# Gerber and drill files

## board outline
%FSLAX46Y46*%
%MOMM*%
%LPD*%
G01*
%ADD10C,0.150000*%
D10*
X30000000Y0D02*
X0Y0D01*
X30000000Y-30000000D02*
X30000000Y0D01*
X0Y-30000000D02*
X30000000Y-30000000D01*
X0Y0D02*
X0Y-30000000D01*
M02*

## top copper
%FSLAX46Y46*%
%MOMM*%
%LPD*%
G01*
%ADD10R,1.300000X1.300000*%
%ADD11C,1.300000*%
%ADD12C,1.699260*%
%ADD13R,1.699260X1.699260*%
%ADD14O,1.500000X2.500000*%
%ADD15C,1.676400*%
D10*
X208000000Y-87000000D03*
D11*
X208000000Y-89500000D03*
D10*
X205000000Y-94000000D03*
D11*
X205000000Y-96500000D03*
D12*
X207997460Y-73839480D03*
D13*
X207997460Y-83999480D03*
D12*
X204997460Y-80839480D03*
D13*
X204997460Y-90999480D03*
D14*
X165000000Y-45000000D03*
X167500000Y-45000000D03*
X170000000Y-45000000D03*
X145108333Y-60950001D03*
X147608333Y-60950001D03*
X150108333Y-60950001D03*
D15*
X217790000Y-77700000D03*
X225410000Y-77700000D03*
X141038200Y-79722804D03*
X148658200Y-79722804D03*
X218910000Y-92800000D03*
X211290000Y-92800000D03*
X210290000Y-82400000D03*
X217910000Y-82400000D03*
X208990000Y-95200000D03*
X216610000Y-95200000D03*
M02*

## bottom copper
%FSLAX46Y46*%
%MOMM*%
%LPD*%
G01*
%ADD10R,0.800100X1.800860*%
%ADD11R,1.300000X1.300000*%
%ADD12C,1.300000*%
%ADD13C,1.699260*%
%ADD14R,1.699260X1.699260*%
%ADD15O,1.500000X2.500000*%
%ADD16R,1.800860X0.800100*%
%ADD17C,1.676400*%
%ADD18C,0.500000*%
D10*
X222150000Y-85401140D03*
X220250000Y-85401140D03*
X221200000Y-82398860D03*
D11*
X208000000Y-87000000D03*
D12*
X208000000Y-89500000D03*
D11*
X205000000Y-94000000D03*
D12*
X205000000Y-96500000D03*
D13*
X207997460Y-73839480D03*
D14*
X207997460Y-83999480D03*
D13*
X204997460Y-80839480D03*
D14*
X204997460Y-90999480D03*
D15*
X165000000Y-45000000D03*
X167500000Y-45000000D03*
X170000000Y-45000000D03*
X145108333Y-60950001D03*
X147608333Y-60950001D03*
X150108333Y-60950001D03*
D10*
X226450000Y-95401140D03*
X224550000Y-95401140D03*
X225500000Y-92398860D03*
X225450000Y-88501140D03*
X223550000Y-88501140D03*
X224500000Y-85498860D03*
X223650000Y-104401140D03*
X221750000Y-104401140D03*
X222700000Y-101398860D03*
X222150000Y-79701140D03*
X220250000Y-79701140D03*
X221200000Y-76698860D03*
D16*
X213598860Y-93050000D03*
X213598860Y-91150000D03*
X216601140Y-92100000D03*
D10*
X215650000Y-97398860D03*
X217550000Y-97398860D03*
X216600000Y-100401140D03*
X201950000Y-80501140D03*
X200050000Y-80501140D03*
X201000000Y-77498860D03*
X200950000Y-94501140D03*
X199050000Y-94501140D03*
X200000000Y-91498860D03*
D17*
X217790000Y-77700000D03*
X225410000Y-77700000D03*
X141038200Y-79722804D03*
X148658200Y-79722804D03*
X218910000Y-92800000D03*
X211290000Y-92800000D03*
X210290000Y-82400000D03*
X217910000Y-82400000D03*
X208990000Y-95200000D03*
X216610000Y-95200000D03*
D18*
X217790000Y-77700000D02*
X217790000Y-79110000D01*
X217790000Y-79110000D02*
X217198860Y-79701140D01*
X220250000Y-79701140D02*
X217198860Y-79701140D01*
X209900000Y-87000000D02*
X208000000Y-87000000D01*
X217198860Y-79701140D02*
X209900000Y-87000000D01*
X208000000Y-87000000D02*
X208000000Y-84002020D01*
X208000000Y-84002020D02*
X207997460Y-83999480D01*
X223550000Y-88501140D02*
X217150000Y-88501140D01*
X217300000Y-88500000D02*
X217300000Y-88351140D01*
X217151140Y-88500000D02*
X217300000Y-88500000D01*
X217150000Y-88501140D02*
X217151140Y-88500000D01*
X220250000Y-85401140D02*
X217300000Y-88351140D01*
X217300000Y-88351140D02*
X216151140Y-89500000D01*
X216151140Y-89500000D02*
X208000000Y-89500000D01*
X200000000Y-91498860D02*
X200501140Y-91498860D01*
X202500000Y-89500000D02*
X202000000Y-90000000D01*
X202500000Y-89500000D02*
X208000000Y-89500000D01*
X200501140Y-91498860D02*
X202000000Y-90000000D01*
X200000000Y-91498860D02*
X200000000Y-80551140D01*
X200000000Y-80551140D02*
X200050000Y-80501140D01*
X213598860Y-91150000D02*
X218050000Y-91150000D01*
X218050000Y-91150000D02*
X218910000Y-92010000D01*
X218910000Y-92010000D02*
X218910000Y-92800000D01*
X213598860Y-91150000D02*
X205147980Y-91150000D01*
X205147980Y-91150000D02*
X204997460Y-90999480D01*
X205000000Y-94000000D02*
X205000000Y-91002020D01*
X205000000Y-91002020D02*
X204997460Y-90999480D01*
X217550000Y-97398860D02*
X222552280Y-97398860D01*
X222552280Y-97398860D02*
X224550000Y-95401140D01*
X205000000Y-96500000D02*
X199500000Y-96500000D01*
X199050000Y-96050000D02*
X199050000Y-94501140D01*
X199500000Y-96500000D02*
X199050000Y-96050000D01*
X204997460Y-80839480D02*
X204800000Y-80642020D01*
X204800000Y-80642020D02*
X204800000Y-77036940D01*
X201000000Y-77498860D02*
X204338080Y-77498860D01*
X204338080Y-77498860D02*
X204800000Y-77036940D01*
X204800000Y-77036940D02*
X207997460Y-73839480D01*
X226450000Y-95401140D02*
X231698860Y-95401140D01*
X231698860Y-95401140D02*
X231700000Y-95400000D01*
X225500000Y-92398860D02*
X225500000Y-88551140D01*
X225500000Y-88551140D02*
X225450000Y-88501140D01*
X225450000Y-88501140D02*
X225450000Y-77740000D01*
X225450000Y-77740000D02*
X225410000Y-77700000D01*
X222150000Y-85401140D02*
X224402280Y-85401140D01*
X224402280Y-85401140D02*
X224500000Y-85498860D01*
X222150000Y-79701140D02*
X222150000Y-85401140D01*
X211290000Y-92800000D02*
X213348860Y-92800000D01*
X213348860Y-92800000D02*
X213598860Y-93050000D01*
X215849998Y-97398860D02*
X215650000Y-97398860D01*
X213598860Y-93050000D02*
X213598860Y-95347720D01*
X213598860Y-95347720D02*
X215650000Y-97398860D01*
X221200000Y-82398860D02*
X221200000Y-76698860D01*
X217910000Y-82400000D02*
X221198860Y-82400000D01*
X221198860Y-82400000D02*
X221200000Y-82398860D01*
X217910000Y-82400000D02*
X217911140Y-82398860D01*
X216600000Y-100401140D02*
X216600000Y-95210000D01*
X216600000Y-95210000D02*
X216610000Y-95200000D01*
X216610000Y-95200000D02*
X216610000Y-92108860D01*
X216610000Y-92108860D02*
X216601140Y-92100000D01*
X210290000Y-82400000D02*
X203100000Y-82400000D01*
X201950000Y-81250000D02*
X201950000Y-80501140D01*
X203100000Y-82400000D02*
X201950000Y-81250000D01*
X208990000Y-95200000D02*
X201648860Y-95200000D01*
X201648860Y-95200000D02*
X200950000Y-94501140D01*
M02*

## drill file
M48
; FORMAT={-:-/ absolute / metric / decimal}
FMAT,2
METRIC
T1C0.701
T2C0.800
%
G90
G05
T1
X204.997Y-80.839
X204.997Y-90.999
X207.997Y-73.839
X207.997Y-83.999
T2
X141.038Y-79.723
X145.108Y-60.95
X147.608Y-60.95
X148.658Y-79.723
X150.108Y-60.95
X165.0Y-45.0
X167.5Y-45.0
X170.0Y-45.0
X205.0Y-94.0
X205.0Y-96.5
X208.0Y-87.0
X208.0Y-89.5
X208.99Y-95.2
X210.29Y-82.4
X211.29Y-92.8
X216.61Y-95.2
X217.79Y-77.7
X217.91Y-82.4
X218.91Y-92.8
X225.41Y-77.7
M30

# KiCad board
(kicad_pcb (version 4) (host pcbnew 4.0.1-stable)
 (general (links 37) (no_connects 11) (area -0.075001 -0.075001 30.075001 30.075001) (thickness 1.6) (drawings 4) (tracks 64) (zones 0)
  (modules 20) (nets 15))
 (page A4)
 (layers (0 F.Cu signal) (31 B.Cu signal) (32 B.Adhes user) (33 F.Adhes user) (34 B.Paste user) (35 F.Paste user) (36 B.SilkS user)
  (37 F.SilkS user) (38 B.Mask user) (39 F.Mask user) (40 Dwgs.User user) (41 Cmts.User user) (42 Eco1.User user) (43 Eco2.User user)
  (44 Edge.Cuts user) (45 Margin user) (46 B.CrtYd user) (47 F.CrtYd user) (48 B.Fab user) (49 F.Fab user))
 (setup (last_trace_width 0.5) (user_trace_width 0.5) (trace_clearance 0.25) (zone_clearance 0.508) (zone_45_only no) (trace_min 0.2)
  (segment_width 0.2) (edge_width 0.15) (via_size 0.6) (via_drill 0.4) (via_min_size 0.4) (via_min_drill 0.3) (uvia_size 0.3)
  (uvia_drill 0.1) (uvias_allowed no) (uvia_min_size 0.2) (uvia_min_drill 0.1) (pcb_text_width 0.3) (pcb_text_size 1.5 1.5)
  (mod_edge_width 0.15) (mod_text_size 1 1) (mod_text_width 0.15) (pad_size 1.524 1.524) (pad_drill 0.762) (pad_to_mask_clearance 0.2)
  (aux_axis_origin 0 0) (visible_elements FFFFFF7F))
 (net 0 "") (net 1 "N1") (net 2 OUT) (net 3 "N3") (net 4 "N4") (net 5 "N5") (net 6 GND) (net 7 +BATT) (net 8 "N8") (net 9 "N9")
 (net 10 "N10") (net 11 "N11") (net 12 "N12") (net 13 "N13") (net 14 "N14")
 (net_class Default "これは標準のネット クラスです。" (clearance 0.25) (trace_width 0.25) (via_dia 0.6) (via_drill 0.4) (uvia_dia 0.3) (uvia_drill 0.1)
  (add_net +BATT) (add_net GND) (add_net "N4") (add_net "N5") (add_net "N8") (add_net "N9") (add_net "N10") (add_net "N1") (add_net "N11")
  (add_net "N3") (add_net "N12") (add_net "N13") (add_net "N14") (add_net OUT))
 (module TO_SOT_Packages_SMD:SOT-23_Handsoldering (layer B.Cu) (at 221.2 83.9 180)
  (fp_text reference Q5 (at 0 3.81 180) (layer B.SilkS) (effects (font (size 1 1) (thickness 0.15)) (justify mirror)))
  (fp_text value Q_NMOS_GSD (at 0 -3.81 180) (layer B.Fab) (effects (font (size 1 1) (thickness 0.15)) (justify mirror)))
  (pad 1 smd rect (at -0.95 -1.50114 180) (size 0.8001 1.80086) (layers B.Cu B.Paste B.Mask) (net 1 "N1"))
  (pad 2 smd rect (at 0.95 -1.50114 180) (size 0.8001 1.80086) (layers B.Cu B.Paste B.Mask) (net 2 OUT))
  (pad 3 smd rect (at 0 1.50114 180) (size 0.8001 1.80086) (layers B.Cu B.Paste B.Mask) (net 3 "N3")))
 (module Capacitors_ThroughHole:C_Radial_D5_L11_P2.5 (layer F.Cu) (at 208 87 270)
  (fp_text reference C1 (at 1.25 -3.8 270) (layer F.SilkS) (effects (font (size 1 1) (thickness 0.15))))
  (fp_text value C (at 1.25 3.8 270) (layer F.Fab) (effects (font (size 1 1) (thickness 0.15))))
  (pad 1 thru_hole rect (at 0 0 270) (size 1.3 1.3) (drill 0.8) (layers *.Cu *.Mask F.SilkS) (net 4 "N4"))
  (pad 2 thru_hole circle (at 2.5 0 270) (size 1.3 1.3) (drill 0.8) (layers *.Cu *.Mask F.SilkS) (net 2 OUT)))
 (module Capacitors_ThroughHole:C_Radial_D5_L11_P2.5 (layer F.Cu) (at 205 94 270)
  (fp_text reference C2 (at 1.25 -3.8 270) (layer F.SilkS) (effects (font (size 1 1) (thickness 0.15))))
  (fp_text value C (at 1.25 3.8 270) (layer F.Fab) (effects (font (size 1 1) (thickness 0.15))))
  (pad 1 thru_hole rect (at 0 0 270) (size 1.3 1.3) (drill 0.8) (layers *.Cu *.Mask F.SilkS) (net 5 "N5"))
  (pad 2 thru_hole circle (at 2.5 0 270) (size 1.3 1.3) (drill 0.8) (layers *.Cu *.Mask F.SilkS) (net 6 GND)))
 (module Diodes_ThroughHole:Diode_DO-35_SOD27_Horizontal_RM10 (layer F.Cu) (at 208 84 90)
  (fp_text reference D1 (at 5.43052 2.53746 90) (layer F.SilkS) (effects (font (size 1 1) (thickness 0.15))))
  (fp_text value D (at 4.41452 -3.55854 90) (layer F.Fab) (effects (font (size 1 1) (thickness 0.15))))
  (pad 2 thru_hole circle (at 10.16052 -0.00254 270) (size 1.69926 1.69926) (drill 0.70104) (layers *.Cu *.Mask F.SilkS) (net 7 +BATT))
  (pad 1 thru_hole rect (at 0.00052 -0.00254 270) (size 1.69926 1.69926) (drill 0.70104) (layers *.Cu *.Mask F.SilkS) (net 4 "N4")))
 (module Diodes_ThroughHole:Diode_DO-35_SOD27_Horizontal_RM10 (layer F.Cu) (at 205 91 90)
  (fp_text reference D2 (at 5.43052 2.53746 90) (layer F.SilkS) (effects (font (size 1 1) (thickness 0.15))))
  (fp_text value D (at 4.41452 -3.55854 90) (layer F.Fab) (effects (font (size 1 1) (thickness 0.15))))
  (pad 2 thru_hole circle (at 10.16052 -0.00254 270) (size 1.69926 1.69926) (drill 0.70104) (layers *.Cu *.Mask F.SilkS) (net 7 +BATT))
  (pad 1 thru_hole rect (at 0.00052 -0.00254 270) (size 1.69926 1.69926) (drill 0.70104) (layers *.Cu *.Mask F.SilkS) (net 5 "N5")))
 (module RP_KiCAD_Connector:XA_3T (layer F.Cu) (at 165 45)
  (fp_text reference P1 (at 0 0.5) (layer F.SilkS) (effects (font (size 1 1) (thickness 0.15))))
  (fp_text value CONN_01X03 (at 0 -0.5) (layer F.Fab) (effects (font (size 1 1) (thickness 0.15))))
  (pad 1 thru_hole oval (at 0 0) (size 1.5 2.5) (drill 0.8) (layers *.Cu *.Mask F.SilkS) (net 6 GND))
  (pad 2 thru_hole oval (at 2.5 0) (size 1.5 2.5) (drill 0.8) (layers *.Cu *.Mask F.SilkS) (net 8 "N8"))
  (pad 3 thru_hole oval (at 5 0) (size 1.5 2.5) (drill 0.8) (layers *.Cu *.Mask F.SilkS) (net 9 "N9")))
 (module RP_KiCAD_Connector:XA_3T (layer F.Cu) (at 145.108333 60.950001)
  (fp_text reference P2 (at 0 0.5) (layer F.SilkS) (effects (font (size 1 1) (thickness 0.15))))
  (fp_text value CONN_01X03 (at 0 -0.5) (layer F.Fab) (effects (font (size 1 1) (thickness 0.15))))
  (pad 1 thru_hole oval (at 0 0) (size 1.5 2.5) (drill 0.8) (layers *.Cu *.Mask F.SilkS) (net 6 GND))
  (pad 2 thru_hole oval (at 2.5 0) (size 1.5 2.5) (drill 0.8) (layers *.Cu *.Mask F.SilkS) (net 7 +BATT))
  (pad 3 thru_hole oval (at 5 0) (size 1.5 2.5) (drill 0.8) (layers *.Cu *.Mask F.SilkS) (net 2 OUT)))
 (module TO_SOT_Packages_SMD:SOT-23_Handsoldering (layer B.Cu) (at 225.5 93.9 180)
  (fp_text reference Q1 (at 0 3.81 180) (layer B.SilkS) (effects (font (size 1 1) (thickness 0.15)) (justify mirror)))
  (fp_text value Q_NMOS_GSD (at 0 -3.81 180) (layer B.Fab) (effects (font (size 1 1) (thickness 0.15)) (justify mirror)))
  (pad 1 smd rect (at -0.95 -1.50114 180) (size 0.8001 1.80086) (layers B.Cu B.Paste B.Mask) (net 9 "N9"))
  (pad 2 smd rect (at 0.95 -1.50114 180) (size 0.8001 1.80086) (layers B.Cu B.Paste B.Mask) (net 6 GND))
  (pad 3 smd rect (at 0 1.50114 180) (size 0.8001 1.80086) (layers B.Cu B.Paste B.Mask) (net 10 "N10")))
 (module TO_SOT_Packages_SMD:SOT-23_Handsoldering (layer B.Cu) (at 224.5 87 180)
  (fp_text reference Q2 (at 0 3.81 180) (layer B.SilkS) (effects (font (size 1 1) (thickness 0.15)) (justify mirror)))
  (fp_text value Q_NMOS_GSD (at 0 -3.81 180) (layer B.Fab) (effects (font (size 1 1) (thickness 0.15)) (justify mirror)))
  (pad 1 smd rect (at -0.95 -1.50114 180) (size 0.8001 1.80086) (layers B.Cu B.Paste B.Mask) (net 10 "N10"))
  (pad 2 smd rect (at 0.95 -1.50114 180) (size 0.8001 1.80086) (layers B.Cu B.Paste B.Mask) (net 2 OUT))
  (pad 3 smd rect (at 0 1.50114 180) (size 0.8001 1.80086) (layers B.Cu B.Paste B.Mask) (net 1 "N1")))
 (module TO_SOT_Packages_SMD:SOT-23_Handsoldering (layer B.Cu) (at 222.7 102.9 180)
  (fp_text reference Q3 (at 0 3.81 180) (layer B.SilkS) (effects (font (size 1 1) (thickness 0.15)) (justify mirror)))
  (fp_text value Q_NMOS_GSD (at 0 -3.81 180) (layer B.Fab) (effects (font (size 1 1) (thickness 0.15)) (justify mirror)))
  (pad 1 smd rect (at -0.95 -1.50114 180) (size 0.8001 1.80086) (layers B.Cu B.Paste B.Mask) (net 8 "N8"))
  (pad 2 smd rect (at 0.95 -1.50114 180) (size 0.8001 1.80086) (layers B.Cu B.Paste B.Mask) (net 6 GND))
  (pad 3 smd rect (at 0 1.50114 180) (size 0.8001 1.80086) (layers B.Cu B.Paste B.Mask) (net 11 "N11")))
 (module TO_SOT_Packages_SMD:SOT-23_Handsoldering (layer B.Cu) (at 221.2 78.2 180)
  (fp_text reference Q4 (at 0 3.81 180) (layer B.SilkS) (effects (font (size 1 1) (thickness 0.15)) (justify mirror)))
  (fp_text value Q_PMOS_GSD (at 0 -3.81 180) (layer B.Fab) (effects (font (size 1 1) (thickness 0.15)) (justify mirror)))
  (pad 1 smd rect (at -0.95 -1.50114 180) (size 0.8001 1.80086) (layers B.Cu B.Paste B.Mask) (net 1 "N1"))
  (pad 2 smd rect (at 0.95 -1.50114 180) (size 0.8001 1.80086) (layers B.Cu B.Paste B.Mask) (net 4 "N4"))
  (pad 3 smd rect (at 0 1.50114 180) (size 0.8001 1.80086) (layers B.Cu B.Paste B.Mask) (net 3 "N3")))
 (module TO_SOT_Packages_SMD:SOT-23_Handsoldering (layer B.Cu) (at 215.1 92.1 90)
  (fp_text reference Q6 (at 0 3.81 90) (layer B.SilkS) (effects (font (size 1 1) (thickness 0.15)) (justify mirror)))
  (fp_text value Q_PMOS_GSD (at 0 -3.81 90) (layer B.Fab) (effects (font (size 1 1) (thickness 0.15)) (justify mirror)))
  (pad 1 smd rect (at -0.95 -1.50114 90) (size 0.8001 1.80086) (layers B.Cu B.Paste B.Mask) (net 11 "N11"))
  (pad 2 smd rect (at 0.95 -1.50114 90) (size 0.8001 1.80086) (layers B.Cu B.Paste B.Mask) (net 5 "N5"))
  (pad 3 smd rect (at 0 1.50114 90) (size 0.8001 1.80086) (layers B.Cu B.Paste B.Mask) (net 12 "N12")))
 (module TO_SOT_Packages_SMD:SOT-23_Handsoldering (layer B.Cu) (at 216.6 98.9)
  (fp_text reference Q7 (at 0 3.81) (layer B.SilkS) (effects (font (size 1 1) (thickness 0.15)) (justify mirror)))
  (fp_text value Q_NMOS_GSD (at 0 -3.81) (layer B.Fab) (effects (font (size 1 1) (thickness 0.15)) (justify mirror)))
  (pad 1 smd rect (at -0.95 -1.50114) (size 0.8001 1.80086) (layers B.Cu B.Paste B.Mask) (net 11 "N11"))
  (pad 2 smd rect (at 0.95 -1.50114) (size 0.8001 1.80086) (layers B.Cu B.Paste B.Mask) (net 6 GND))
  (pad 3 smd rect (at 0 1.50114) (size 0.8001 1.80086) (layers B.Cu B.Paste B.Mask) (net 12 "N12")))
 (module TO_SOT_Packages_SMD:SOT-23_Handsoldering (layer B.Cu) (at 201 79 180)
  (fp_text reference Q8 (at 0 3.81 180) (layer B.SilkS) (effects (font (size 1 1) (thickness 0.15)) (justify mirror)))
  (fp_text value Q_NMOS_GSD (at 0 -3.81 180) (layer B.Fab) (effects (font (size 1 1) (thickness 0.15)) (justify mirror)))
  (pad 1 smd rect (at -0.95 -1.50114 180) (size 0.8001 1.80086) (layers B.Cu B.Paste B.Mask) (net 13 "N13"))
  (pad 2 smd rect (at 0.95 -1.50114 180) (size 0.8001 1.80086) (layers B.Cu B.Paste B.Mask) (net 2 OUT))
  (pad 3 smd rect (at 0 1.50114 180) (size 0.8001 1.80086) (layers B.Cu B.Paste B.Mask) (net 7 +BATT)))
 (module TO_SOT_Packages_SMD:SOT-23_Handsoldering (layer B.Cu) (at 200 93 180)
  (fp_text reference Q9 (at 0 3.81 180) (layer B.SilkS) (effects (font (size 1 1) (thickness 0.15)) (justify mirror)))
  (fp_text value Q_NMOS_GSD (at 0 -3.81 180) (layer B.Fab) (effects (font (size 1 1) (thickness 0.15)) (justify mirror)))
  (pad 1 smd rect (at -0.95 -1.50114 180) (size 0.8001 1.80086) (layers B.Cu B.Paste B.Mask) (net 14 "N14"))
  (pad 2 smd rect (at 0.95 -1.50114 180) (size 0.8001 1.80086) (layers B.Cu B.Paste B.Mask) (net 6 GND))
  (pad 3 smd rect (at 0 1.50114 180) (size 0.8001 1.80086) (layers B.Cu B.Paste B.Mask) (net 2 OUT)))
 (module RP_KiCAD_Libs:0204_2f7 (layer F.Cu) (at 221.6 77.7)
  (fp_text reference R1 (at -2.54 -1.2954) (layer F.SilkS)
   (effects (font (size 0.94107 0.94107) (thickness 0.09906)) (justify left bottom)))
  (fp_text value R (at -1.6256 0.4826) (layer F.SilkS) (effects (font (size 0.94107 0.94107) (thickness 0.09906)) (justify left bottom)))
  (pad 1 thru_hole circle (at -3.81 0) (size 1.6764 1.6764) (drill 0.8) (layers *.Cu *.Mask) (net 4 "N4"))
  (pad 2 thru_hole circle (at 3.81 0) (size 1.6764 1.6764) (drill 0.8) (layers *.Cu *.Mask) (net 10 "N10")))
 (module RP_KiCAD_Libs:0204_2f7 (layer F.Cu) (at 144.8482 79.722804)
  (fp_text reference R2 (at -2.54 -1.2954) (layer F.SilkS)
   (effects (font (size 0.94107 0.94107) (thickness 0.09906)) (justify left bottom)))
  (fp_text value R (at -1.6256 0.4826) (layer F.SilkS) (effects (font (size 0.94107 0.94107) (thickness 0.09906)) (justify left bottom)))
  (pad 1 thru_hole circle (at -3.81 0) (size 1.6764 1.6764) (drill 0.8) (layers *.Cu *.Mask) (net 4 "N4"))
  (pad 2 thru_hole circle (at 3.81 0) (size 1.6764 1.6764) (drill 0.8) (layers *.Cu *.Mask) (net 1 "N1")))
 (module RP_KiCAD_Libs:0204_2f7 (layer F.Cu) (at 215.1 92.8 180)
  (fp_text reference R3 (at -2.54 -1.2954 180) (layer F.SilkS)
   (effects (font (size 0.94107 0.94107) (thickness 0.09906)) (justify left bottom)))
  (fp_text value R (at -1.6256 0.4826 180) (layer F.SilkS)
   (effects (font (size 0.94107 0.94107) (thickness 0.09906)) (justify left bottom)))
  (pad 1 thru_hole circle (at -3.81 0 180) (size 1.6764 1.6764) (drill 0.8) (layers *.Cu *.Mask) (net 5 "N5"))
  (pad 2 thru_hole circle (at 3.81 0 180) (size 1.6764 1.6764) (drill 0.8) (layers *.Cu *.Mask) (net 11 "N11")))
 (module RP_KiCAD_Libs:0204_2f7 (layer F.Cu) (at 214.1 82.4)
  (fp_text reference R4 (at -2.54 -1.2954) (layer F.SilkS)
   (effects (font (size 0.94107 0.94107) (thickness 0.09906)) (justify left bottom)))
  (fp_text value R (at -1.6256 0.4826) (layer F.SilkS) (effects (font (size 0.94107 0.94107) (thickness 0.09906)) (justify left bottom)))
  (pad 1 thru_hole circle (at -3.81 0) (size 1.6764 1.6764) (drill 0.8) (layers *.Cu *.Mask) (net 13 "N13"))
  (pad 2 thru_hole circle (at 3.81 0) (size 1.6764 1.6764) (drill 0.8) (layers *.Cu *.Mask) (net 3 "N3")))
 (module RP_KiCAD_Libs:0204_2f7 (layer F.Cu) (at 212.8 95.2)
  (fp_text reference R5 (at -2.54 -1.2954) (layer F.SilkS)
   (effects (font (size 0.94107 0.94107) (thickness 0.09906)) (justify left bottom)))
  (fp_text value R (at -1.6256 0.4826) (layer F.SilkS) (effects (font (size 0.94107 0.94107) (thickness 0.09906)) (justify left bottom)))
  (pad 1 thru_hole circle (at -3.81 0) (size 1.6764 1.6764) (drill 0.8) (layers *.Cu *.Mask) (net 14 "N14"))
  (pad 2 thru_hole circle (at 3.81 0) (size 1.6764 1.6764) (drill 0.8) (layers *.Cu *.Mask) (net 12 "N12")))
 (gr_line (start 30 0) (end 0 0) (angle 90) (layer Edge.Cuts) (width 0.15))
 (gr_line (start 30 30) (end 30 0) (angle 90) (layer Edge.Cuts) (width 0.15))
 (gr_line (start 0 30) (end 30 30) (angle 90) (layer Edge.Cuts) (width 0.15))
 (gr_line (start 0 0) (end 0 30) (angle 90) (layer Edge.Cuts) (width 0.15))
 (segment (start 217.79 77.7) (end 217.79 79.11) (width 0.5) (layer B.Cu) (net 4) (status 400000))
 (segment (start 217.79 79.11) (end 217.19886 79.70114) (width 0.5) (layer B.Cu) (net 4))
 (segment (start 220.25 79.70114) (end 217.19886 79.70114) (width 0.5) (layer B.Cu) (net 4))
 (segment (start 209.9 87) (end 208 87) (width 0.5) (layer B.Cu) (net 4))
 (segment (start 217.19886 79.70114) (end 209.9 87) (width 0.5) (layer B.Cu) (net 4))
 (segment (start 208 87) (end 208 84.00202) (width 0.5) (layer B.Cu) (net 4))
 (segment (start 208 84.00202) (end 207.99746 83.99948) (width 0.5) (layer B.Cu) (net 4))
 (segment (start 223.55 88.50114) (end 217.15 88.50114) (width 0.5) (layer B.Cu) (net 2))
 (segment (start 217.3 88.5) (end 217.3 88.35114) (width 0.5) (layer B.Cu) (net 2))
 (segment (start 217.15114 88.5) (end 217.3 88.5) (width 0.5) (layer B.Cu) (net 2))
 (segment (start 217.15 88.50114) (end 217.15114 88.5) (width 0.5) (layer B.Cu) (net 2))
 (segment (start 220.25 85.40114) (end 217.3 88.35114) (width 0.5) (layer B.Cu) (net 2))
 (segment (start 217.3 88.35114) (end 216.15114 89.5) (width 0.5) (layer B.Cu) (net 2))
 (segment (start 216.15114 89.5) (end 208 89.5) (width 0.5) (layer B.Cu) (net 2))
 (segment (start 200 91.49886) (end 200.50114 91.49886) (width 0.5) (layer B.Cu) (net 2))
 (segment (start 202.5 89.5) (end 202 90) (width 0.5) (layer B.Cu) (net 2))
 (segment (start 202.5 89.5) (end 208 89.5) (width 0.5) (layer B.Cu) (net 2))
 (segment (start 200.50114 91.49886) (end 202 90) (width 0.5) (layer B.Cu) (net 2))
 (segment (start 200 91.49886) (end 200 80.55114) (width 0.5) (layer B.Cu) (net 2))
 (segment (start 200 80.55114) (end 200.05 80.50114) (width 0.5) (layer B.Cu) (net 2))
 (segment (start 213.59886 91.15) (end 218.05 91.15) (width 0.5) (layer B.Cu) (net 5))
 (segment (start 218.05 91.15) (end 218.91 92.01) (width 0.5) (layer B.Cu) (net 5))
 (segment (start 218.91 92.01) (end 218.91 92.8) (width 0.5) (layer B.Cu) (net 5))
 (segment (start 213.59886 91.15) (end 205.14798 91.15) (width 0.5) (layer B.Cu) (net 5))
 (segment (start 205.14798 91.15) (end 204.99746 90.99948) (width 0.5) (layer B.Cu) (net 5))
 (segment (start 205 94) (end 205 91.00202) (width 0.5) (layer B.Cu) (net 5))
 (segment (start 205 91.00202) (end 204.99746 90.99948) (width 0.5) (layer B.Cu) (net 5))
 (segment (start 217.55 97.39886) (end 222.55228 97.39886) (width 0.5) (layer B.Cu) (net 6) (status 400000))
 (segment (start 222.55228 97.39886) (end 224.55 95.40114) (width 0.5) (layer B.Cu) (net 6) (status 800000))
 (segment (start 205 96.5) (end 199.5 96.5) (width 0.5) (layer B.Cu) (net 6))
 (segment (start 199.05 96.05) (end 199.05 94.50114) (width 0.5) (layer B.Cu) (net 6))
 (segment (start 199.5 96.5) (end 199.05 96.05) (width 0.5) (layer B.Cu) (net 6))
 (segment (start 204.99746 80.83948) (end 204.8 80.64202) (width 0.5) (layer B.Cu) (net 7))
 (segment (start 204.8 80.64202) (end 204.8 77.03694) (width 0.5) (layer B.Cu) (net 7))
 (segment (start 201 77.49886) (end 204.33808 77.49886) (width 0.5) (layer B.Cu) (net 7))
 (segment (start 204.33808 77.49886) (end 204.8 77.03694) (width 0.5) (layer B.Cu) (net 7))
 (segment (start 204.8 77.03694) (end 207.99746 73.83948) (width 0.5) (layer B.Cu) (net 7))
 (segment (start 226.45 95.40114) (end 231.69886 95.40114) (width 0.5) (layer B.Cu) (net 9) (status 400000))
 (segment (start 231.69886 95.40114) (end 231.7 95.4) (width 0.5) (layer B.Cu) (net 9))
 (segment (start 225.5 92.39886) (end 225.5 88.55114) (width 0.5) (layer B.Cu) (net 10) (status C00000))
 (segment (start 225.5 88.55114) (end 225.45 88.50114) (width 0.5) (layer B.Cu) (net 10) (status C00000))
 (segment (start 225.45 88.50114) (end 225.45 77.74) (width 0.5) (layer B.Cu) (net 10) (status C00000))
 (segment (start 225.45 77.74) (end 225.41 77.7) (width 0.5) (layer B.Cu) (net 10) (status C00000))
 (segment (start 222.15 85.40114) (end 224.40228 85.40114) (width 0.5) (layer B.Cu) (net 1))
 (segment (start 224.40228 85.40114) (end 224.5 85.49886) (width 0.5) (layer B.Cu) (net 1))
 (segment (start 222.15 79.70114) (end 222.15 85.40114) (width 0.5) (layer B.Cu) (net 1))
 (segment (start 211.29 92.8) (end 213.34886 92.8) (width 0.5) (layer B.Cu) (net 11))
 (segment (start 213.34886 92.8) (end 213.59886 93.05) (width 0.5) (layer B.Cu) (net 11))
 (segment (start 215.849998 97.39886) (end 215.65 97.39886) (width 0.5) (layer B.Cu) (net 11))
 (segment (start 213.59886 93.05) (end 213.59886 95.34772) (width 0.5) (layer B.Cu) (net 11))
 (segment (start 213.59886 95.34772) (end 215.65 97.39886) (width 0.5) (layer B.Cu) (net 11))
 (segment (start 221.2 82.39886) (end 221.2 76.69886) (width 0.5) (layer B.Cu) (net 3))
 (segment (start 217.91 82.4) (end 221.19886 82.4) (width 0.5) (layer B.Cu) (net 3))
 (segment (start 221.19886 82.4) (end 221.2 82.39886) (width 0.5) (layer B.Cu) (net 3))
 (segment (start 217.91 82.4) (end 217.91114 82.39886) (width 0.5) (layer B.Cu) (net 3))
 (segment (start 216.6 100.40114) (end 216.6 95.21) (width 0.5) (layer B.Cu) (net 12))
 (segment (start 216.6 95.21) (end 216.61 95.2) (width 0.5) (layer B.Cu) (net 12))
 (segment (start 216.61 95.2) (end 216.61 92.10886) (width 0.5) (layer B.Cu) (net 12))
 (segment (start 216.61 92.10886) (end 216.60114 92.1) (width 0.5) (layer B.Cu) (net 12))
 (segment (start 210.29 82.4) (end 203.1 82.4) (width 0.5) (layer B.Cu) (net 13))
 (segment (start 201.95 81.25) (end 201.95 80.50114) (width 0.5) (layer B.Cu) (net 13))
 (segment (start 203.1 82.4) (end 201.95 81.25) (width 0.5) (layer B.Cu) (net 13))
 (segment (start 208.99 95.2) (end 201.64886 95.2) (width 0.5) (layer B.Cu) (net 14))
 (segment (start 201.64886 95.2) (end 200.95 94.50114) (width 0.5) (layer B.Cu) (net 14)))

